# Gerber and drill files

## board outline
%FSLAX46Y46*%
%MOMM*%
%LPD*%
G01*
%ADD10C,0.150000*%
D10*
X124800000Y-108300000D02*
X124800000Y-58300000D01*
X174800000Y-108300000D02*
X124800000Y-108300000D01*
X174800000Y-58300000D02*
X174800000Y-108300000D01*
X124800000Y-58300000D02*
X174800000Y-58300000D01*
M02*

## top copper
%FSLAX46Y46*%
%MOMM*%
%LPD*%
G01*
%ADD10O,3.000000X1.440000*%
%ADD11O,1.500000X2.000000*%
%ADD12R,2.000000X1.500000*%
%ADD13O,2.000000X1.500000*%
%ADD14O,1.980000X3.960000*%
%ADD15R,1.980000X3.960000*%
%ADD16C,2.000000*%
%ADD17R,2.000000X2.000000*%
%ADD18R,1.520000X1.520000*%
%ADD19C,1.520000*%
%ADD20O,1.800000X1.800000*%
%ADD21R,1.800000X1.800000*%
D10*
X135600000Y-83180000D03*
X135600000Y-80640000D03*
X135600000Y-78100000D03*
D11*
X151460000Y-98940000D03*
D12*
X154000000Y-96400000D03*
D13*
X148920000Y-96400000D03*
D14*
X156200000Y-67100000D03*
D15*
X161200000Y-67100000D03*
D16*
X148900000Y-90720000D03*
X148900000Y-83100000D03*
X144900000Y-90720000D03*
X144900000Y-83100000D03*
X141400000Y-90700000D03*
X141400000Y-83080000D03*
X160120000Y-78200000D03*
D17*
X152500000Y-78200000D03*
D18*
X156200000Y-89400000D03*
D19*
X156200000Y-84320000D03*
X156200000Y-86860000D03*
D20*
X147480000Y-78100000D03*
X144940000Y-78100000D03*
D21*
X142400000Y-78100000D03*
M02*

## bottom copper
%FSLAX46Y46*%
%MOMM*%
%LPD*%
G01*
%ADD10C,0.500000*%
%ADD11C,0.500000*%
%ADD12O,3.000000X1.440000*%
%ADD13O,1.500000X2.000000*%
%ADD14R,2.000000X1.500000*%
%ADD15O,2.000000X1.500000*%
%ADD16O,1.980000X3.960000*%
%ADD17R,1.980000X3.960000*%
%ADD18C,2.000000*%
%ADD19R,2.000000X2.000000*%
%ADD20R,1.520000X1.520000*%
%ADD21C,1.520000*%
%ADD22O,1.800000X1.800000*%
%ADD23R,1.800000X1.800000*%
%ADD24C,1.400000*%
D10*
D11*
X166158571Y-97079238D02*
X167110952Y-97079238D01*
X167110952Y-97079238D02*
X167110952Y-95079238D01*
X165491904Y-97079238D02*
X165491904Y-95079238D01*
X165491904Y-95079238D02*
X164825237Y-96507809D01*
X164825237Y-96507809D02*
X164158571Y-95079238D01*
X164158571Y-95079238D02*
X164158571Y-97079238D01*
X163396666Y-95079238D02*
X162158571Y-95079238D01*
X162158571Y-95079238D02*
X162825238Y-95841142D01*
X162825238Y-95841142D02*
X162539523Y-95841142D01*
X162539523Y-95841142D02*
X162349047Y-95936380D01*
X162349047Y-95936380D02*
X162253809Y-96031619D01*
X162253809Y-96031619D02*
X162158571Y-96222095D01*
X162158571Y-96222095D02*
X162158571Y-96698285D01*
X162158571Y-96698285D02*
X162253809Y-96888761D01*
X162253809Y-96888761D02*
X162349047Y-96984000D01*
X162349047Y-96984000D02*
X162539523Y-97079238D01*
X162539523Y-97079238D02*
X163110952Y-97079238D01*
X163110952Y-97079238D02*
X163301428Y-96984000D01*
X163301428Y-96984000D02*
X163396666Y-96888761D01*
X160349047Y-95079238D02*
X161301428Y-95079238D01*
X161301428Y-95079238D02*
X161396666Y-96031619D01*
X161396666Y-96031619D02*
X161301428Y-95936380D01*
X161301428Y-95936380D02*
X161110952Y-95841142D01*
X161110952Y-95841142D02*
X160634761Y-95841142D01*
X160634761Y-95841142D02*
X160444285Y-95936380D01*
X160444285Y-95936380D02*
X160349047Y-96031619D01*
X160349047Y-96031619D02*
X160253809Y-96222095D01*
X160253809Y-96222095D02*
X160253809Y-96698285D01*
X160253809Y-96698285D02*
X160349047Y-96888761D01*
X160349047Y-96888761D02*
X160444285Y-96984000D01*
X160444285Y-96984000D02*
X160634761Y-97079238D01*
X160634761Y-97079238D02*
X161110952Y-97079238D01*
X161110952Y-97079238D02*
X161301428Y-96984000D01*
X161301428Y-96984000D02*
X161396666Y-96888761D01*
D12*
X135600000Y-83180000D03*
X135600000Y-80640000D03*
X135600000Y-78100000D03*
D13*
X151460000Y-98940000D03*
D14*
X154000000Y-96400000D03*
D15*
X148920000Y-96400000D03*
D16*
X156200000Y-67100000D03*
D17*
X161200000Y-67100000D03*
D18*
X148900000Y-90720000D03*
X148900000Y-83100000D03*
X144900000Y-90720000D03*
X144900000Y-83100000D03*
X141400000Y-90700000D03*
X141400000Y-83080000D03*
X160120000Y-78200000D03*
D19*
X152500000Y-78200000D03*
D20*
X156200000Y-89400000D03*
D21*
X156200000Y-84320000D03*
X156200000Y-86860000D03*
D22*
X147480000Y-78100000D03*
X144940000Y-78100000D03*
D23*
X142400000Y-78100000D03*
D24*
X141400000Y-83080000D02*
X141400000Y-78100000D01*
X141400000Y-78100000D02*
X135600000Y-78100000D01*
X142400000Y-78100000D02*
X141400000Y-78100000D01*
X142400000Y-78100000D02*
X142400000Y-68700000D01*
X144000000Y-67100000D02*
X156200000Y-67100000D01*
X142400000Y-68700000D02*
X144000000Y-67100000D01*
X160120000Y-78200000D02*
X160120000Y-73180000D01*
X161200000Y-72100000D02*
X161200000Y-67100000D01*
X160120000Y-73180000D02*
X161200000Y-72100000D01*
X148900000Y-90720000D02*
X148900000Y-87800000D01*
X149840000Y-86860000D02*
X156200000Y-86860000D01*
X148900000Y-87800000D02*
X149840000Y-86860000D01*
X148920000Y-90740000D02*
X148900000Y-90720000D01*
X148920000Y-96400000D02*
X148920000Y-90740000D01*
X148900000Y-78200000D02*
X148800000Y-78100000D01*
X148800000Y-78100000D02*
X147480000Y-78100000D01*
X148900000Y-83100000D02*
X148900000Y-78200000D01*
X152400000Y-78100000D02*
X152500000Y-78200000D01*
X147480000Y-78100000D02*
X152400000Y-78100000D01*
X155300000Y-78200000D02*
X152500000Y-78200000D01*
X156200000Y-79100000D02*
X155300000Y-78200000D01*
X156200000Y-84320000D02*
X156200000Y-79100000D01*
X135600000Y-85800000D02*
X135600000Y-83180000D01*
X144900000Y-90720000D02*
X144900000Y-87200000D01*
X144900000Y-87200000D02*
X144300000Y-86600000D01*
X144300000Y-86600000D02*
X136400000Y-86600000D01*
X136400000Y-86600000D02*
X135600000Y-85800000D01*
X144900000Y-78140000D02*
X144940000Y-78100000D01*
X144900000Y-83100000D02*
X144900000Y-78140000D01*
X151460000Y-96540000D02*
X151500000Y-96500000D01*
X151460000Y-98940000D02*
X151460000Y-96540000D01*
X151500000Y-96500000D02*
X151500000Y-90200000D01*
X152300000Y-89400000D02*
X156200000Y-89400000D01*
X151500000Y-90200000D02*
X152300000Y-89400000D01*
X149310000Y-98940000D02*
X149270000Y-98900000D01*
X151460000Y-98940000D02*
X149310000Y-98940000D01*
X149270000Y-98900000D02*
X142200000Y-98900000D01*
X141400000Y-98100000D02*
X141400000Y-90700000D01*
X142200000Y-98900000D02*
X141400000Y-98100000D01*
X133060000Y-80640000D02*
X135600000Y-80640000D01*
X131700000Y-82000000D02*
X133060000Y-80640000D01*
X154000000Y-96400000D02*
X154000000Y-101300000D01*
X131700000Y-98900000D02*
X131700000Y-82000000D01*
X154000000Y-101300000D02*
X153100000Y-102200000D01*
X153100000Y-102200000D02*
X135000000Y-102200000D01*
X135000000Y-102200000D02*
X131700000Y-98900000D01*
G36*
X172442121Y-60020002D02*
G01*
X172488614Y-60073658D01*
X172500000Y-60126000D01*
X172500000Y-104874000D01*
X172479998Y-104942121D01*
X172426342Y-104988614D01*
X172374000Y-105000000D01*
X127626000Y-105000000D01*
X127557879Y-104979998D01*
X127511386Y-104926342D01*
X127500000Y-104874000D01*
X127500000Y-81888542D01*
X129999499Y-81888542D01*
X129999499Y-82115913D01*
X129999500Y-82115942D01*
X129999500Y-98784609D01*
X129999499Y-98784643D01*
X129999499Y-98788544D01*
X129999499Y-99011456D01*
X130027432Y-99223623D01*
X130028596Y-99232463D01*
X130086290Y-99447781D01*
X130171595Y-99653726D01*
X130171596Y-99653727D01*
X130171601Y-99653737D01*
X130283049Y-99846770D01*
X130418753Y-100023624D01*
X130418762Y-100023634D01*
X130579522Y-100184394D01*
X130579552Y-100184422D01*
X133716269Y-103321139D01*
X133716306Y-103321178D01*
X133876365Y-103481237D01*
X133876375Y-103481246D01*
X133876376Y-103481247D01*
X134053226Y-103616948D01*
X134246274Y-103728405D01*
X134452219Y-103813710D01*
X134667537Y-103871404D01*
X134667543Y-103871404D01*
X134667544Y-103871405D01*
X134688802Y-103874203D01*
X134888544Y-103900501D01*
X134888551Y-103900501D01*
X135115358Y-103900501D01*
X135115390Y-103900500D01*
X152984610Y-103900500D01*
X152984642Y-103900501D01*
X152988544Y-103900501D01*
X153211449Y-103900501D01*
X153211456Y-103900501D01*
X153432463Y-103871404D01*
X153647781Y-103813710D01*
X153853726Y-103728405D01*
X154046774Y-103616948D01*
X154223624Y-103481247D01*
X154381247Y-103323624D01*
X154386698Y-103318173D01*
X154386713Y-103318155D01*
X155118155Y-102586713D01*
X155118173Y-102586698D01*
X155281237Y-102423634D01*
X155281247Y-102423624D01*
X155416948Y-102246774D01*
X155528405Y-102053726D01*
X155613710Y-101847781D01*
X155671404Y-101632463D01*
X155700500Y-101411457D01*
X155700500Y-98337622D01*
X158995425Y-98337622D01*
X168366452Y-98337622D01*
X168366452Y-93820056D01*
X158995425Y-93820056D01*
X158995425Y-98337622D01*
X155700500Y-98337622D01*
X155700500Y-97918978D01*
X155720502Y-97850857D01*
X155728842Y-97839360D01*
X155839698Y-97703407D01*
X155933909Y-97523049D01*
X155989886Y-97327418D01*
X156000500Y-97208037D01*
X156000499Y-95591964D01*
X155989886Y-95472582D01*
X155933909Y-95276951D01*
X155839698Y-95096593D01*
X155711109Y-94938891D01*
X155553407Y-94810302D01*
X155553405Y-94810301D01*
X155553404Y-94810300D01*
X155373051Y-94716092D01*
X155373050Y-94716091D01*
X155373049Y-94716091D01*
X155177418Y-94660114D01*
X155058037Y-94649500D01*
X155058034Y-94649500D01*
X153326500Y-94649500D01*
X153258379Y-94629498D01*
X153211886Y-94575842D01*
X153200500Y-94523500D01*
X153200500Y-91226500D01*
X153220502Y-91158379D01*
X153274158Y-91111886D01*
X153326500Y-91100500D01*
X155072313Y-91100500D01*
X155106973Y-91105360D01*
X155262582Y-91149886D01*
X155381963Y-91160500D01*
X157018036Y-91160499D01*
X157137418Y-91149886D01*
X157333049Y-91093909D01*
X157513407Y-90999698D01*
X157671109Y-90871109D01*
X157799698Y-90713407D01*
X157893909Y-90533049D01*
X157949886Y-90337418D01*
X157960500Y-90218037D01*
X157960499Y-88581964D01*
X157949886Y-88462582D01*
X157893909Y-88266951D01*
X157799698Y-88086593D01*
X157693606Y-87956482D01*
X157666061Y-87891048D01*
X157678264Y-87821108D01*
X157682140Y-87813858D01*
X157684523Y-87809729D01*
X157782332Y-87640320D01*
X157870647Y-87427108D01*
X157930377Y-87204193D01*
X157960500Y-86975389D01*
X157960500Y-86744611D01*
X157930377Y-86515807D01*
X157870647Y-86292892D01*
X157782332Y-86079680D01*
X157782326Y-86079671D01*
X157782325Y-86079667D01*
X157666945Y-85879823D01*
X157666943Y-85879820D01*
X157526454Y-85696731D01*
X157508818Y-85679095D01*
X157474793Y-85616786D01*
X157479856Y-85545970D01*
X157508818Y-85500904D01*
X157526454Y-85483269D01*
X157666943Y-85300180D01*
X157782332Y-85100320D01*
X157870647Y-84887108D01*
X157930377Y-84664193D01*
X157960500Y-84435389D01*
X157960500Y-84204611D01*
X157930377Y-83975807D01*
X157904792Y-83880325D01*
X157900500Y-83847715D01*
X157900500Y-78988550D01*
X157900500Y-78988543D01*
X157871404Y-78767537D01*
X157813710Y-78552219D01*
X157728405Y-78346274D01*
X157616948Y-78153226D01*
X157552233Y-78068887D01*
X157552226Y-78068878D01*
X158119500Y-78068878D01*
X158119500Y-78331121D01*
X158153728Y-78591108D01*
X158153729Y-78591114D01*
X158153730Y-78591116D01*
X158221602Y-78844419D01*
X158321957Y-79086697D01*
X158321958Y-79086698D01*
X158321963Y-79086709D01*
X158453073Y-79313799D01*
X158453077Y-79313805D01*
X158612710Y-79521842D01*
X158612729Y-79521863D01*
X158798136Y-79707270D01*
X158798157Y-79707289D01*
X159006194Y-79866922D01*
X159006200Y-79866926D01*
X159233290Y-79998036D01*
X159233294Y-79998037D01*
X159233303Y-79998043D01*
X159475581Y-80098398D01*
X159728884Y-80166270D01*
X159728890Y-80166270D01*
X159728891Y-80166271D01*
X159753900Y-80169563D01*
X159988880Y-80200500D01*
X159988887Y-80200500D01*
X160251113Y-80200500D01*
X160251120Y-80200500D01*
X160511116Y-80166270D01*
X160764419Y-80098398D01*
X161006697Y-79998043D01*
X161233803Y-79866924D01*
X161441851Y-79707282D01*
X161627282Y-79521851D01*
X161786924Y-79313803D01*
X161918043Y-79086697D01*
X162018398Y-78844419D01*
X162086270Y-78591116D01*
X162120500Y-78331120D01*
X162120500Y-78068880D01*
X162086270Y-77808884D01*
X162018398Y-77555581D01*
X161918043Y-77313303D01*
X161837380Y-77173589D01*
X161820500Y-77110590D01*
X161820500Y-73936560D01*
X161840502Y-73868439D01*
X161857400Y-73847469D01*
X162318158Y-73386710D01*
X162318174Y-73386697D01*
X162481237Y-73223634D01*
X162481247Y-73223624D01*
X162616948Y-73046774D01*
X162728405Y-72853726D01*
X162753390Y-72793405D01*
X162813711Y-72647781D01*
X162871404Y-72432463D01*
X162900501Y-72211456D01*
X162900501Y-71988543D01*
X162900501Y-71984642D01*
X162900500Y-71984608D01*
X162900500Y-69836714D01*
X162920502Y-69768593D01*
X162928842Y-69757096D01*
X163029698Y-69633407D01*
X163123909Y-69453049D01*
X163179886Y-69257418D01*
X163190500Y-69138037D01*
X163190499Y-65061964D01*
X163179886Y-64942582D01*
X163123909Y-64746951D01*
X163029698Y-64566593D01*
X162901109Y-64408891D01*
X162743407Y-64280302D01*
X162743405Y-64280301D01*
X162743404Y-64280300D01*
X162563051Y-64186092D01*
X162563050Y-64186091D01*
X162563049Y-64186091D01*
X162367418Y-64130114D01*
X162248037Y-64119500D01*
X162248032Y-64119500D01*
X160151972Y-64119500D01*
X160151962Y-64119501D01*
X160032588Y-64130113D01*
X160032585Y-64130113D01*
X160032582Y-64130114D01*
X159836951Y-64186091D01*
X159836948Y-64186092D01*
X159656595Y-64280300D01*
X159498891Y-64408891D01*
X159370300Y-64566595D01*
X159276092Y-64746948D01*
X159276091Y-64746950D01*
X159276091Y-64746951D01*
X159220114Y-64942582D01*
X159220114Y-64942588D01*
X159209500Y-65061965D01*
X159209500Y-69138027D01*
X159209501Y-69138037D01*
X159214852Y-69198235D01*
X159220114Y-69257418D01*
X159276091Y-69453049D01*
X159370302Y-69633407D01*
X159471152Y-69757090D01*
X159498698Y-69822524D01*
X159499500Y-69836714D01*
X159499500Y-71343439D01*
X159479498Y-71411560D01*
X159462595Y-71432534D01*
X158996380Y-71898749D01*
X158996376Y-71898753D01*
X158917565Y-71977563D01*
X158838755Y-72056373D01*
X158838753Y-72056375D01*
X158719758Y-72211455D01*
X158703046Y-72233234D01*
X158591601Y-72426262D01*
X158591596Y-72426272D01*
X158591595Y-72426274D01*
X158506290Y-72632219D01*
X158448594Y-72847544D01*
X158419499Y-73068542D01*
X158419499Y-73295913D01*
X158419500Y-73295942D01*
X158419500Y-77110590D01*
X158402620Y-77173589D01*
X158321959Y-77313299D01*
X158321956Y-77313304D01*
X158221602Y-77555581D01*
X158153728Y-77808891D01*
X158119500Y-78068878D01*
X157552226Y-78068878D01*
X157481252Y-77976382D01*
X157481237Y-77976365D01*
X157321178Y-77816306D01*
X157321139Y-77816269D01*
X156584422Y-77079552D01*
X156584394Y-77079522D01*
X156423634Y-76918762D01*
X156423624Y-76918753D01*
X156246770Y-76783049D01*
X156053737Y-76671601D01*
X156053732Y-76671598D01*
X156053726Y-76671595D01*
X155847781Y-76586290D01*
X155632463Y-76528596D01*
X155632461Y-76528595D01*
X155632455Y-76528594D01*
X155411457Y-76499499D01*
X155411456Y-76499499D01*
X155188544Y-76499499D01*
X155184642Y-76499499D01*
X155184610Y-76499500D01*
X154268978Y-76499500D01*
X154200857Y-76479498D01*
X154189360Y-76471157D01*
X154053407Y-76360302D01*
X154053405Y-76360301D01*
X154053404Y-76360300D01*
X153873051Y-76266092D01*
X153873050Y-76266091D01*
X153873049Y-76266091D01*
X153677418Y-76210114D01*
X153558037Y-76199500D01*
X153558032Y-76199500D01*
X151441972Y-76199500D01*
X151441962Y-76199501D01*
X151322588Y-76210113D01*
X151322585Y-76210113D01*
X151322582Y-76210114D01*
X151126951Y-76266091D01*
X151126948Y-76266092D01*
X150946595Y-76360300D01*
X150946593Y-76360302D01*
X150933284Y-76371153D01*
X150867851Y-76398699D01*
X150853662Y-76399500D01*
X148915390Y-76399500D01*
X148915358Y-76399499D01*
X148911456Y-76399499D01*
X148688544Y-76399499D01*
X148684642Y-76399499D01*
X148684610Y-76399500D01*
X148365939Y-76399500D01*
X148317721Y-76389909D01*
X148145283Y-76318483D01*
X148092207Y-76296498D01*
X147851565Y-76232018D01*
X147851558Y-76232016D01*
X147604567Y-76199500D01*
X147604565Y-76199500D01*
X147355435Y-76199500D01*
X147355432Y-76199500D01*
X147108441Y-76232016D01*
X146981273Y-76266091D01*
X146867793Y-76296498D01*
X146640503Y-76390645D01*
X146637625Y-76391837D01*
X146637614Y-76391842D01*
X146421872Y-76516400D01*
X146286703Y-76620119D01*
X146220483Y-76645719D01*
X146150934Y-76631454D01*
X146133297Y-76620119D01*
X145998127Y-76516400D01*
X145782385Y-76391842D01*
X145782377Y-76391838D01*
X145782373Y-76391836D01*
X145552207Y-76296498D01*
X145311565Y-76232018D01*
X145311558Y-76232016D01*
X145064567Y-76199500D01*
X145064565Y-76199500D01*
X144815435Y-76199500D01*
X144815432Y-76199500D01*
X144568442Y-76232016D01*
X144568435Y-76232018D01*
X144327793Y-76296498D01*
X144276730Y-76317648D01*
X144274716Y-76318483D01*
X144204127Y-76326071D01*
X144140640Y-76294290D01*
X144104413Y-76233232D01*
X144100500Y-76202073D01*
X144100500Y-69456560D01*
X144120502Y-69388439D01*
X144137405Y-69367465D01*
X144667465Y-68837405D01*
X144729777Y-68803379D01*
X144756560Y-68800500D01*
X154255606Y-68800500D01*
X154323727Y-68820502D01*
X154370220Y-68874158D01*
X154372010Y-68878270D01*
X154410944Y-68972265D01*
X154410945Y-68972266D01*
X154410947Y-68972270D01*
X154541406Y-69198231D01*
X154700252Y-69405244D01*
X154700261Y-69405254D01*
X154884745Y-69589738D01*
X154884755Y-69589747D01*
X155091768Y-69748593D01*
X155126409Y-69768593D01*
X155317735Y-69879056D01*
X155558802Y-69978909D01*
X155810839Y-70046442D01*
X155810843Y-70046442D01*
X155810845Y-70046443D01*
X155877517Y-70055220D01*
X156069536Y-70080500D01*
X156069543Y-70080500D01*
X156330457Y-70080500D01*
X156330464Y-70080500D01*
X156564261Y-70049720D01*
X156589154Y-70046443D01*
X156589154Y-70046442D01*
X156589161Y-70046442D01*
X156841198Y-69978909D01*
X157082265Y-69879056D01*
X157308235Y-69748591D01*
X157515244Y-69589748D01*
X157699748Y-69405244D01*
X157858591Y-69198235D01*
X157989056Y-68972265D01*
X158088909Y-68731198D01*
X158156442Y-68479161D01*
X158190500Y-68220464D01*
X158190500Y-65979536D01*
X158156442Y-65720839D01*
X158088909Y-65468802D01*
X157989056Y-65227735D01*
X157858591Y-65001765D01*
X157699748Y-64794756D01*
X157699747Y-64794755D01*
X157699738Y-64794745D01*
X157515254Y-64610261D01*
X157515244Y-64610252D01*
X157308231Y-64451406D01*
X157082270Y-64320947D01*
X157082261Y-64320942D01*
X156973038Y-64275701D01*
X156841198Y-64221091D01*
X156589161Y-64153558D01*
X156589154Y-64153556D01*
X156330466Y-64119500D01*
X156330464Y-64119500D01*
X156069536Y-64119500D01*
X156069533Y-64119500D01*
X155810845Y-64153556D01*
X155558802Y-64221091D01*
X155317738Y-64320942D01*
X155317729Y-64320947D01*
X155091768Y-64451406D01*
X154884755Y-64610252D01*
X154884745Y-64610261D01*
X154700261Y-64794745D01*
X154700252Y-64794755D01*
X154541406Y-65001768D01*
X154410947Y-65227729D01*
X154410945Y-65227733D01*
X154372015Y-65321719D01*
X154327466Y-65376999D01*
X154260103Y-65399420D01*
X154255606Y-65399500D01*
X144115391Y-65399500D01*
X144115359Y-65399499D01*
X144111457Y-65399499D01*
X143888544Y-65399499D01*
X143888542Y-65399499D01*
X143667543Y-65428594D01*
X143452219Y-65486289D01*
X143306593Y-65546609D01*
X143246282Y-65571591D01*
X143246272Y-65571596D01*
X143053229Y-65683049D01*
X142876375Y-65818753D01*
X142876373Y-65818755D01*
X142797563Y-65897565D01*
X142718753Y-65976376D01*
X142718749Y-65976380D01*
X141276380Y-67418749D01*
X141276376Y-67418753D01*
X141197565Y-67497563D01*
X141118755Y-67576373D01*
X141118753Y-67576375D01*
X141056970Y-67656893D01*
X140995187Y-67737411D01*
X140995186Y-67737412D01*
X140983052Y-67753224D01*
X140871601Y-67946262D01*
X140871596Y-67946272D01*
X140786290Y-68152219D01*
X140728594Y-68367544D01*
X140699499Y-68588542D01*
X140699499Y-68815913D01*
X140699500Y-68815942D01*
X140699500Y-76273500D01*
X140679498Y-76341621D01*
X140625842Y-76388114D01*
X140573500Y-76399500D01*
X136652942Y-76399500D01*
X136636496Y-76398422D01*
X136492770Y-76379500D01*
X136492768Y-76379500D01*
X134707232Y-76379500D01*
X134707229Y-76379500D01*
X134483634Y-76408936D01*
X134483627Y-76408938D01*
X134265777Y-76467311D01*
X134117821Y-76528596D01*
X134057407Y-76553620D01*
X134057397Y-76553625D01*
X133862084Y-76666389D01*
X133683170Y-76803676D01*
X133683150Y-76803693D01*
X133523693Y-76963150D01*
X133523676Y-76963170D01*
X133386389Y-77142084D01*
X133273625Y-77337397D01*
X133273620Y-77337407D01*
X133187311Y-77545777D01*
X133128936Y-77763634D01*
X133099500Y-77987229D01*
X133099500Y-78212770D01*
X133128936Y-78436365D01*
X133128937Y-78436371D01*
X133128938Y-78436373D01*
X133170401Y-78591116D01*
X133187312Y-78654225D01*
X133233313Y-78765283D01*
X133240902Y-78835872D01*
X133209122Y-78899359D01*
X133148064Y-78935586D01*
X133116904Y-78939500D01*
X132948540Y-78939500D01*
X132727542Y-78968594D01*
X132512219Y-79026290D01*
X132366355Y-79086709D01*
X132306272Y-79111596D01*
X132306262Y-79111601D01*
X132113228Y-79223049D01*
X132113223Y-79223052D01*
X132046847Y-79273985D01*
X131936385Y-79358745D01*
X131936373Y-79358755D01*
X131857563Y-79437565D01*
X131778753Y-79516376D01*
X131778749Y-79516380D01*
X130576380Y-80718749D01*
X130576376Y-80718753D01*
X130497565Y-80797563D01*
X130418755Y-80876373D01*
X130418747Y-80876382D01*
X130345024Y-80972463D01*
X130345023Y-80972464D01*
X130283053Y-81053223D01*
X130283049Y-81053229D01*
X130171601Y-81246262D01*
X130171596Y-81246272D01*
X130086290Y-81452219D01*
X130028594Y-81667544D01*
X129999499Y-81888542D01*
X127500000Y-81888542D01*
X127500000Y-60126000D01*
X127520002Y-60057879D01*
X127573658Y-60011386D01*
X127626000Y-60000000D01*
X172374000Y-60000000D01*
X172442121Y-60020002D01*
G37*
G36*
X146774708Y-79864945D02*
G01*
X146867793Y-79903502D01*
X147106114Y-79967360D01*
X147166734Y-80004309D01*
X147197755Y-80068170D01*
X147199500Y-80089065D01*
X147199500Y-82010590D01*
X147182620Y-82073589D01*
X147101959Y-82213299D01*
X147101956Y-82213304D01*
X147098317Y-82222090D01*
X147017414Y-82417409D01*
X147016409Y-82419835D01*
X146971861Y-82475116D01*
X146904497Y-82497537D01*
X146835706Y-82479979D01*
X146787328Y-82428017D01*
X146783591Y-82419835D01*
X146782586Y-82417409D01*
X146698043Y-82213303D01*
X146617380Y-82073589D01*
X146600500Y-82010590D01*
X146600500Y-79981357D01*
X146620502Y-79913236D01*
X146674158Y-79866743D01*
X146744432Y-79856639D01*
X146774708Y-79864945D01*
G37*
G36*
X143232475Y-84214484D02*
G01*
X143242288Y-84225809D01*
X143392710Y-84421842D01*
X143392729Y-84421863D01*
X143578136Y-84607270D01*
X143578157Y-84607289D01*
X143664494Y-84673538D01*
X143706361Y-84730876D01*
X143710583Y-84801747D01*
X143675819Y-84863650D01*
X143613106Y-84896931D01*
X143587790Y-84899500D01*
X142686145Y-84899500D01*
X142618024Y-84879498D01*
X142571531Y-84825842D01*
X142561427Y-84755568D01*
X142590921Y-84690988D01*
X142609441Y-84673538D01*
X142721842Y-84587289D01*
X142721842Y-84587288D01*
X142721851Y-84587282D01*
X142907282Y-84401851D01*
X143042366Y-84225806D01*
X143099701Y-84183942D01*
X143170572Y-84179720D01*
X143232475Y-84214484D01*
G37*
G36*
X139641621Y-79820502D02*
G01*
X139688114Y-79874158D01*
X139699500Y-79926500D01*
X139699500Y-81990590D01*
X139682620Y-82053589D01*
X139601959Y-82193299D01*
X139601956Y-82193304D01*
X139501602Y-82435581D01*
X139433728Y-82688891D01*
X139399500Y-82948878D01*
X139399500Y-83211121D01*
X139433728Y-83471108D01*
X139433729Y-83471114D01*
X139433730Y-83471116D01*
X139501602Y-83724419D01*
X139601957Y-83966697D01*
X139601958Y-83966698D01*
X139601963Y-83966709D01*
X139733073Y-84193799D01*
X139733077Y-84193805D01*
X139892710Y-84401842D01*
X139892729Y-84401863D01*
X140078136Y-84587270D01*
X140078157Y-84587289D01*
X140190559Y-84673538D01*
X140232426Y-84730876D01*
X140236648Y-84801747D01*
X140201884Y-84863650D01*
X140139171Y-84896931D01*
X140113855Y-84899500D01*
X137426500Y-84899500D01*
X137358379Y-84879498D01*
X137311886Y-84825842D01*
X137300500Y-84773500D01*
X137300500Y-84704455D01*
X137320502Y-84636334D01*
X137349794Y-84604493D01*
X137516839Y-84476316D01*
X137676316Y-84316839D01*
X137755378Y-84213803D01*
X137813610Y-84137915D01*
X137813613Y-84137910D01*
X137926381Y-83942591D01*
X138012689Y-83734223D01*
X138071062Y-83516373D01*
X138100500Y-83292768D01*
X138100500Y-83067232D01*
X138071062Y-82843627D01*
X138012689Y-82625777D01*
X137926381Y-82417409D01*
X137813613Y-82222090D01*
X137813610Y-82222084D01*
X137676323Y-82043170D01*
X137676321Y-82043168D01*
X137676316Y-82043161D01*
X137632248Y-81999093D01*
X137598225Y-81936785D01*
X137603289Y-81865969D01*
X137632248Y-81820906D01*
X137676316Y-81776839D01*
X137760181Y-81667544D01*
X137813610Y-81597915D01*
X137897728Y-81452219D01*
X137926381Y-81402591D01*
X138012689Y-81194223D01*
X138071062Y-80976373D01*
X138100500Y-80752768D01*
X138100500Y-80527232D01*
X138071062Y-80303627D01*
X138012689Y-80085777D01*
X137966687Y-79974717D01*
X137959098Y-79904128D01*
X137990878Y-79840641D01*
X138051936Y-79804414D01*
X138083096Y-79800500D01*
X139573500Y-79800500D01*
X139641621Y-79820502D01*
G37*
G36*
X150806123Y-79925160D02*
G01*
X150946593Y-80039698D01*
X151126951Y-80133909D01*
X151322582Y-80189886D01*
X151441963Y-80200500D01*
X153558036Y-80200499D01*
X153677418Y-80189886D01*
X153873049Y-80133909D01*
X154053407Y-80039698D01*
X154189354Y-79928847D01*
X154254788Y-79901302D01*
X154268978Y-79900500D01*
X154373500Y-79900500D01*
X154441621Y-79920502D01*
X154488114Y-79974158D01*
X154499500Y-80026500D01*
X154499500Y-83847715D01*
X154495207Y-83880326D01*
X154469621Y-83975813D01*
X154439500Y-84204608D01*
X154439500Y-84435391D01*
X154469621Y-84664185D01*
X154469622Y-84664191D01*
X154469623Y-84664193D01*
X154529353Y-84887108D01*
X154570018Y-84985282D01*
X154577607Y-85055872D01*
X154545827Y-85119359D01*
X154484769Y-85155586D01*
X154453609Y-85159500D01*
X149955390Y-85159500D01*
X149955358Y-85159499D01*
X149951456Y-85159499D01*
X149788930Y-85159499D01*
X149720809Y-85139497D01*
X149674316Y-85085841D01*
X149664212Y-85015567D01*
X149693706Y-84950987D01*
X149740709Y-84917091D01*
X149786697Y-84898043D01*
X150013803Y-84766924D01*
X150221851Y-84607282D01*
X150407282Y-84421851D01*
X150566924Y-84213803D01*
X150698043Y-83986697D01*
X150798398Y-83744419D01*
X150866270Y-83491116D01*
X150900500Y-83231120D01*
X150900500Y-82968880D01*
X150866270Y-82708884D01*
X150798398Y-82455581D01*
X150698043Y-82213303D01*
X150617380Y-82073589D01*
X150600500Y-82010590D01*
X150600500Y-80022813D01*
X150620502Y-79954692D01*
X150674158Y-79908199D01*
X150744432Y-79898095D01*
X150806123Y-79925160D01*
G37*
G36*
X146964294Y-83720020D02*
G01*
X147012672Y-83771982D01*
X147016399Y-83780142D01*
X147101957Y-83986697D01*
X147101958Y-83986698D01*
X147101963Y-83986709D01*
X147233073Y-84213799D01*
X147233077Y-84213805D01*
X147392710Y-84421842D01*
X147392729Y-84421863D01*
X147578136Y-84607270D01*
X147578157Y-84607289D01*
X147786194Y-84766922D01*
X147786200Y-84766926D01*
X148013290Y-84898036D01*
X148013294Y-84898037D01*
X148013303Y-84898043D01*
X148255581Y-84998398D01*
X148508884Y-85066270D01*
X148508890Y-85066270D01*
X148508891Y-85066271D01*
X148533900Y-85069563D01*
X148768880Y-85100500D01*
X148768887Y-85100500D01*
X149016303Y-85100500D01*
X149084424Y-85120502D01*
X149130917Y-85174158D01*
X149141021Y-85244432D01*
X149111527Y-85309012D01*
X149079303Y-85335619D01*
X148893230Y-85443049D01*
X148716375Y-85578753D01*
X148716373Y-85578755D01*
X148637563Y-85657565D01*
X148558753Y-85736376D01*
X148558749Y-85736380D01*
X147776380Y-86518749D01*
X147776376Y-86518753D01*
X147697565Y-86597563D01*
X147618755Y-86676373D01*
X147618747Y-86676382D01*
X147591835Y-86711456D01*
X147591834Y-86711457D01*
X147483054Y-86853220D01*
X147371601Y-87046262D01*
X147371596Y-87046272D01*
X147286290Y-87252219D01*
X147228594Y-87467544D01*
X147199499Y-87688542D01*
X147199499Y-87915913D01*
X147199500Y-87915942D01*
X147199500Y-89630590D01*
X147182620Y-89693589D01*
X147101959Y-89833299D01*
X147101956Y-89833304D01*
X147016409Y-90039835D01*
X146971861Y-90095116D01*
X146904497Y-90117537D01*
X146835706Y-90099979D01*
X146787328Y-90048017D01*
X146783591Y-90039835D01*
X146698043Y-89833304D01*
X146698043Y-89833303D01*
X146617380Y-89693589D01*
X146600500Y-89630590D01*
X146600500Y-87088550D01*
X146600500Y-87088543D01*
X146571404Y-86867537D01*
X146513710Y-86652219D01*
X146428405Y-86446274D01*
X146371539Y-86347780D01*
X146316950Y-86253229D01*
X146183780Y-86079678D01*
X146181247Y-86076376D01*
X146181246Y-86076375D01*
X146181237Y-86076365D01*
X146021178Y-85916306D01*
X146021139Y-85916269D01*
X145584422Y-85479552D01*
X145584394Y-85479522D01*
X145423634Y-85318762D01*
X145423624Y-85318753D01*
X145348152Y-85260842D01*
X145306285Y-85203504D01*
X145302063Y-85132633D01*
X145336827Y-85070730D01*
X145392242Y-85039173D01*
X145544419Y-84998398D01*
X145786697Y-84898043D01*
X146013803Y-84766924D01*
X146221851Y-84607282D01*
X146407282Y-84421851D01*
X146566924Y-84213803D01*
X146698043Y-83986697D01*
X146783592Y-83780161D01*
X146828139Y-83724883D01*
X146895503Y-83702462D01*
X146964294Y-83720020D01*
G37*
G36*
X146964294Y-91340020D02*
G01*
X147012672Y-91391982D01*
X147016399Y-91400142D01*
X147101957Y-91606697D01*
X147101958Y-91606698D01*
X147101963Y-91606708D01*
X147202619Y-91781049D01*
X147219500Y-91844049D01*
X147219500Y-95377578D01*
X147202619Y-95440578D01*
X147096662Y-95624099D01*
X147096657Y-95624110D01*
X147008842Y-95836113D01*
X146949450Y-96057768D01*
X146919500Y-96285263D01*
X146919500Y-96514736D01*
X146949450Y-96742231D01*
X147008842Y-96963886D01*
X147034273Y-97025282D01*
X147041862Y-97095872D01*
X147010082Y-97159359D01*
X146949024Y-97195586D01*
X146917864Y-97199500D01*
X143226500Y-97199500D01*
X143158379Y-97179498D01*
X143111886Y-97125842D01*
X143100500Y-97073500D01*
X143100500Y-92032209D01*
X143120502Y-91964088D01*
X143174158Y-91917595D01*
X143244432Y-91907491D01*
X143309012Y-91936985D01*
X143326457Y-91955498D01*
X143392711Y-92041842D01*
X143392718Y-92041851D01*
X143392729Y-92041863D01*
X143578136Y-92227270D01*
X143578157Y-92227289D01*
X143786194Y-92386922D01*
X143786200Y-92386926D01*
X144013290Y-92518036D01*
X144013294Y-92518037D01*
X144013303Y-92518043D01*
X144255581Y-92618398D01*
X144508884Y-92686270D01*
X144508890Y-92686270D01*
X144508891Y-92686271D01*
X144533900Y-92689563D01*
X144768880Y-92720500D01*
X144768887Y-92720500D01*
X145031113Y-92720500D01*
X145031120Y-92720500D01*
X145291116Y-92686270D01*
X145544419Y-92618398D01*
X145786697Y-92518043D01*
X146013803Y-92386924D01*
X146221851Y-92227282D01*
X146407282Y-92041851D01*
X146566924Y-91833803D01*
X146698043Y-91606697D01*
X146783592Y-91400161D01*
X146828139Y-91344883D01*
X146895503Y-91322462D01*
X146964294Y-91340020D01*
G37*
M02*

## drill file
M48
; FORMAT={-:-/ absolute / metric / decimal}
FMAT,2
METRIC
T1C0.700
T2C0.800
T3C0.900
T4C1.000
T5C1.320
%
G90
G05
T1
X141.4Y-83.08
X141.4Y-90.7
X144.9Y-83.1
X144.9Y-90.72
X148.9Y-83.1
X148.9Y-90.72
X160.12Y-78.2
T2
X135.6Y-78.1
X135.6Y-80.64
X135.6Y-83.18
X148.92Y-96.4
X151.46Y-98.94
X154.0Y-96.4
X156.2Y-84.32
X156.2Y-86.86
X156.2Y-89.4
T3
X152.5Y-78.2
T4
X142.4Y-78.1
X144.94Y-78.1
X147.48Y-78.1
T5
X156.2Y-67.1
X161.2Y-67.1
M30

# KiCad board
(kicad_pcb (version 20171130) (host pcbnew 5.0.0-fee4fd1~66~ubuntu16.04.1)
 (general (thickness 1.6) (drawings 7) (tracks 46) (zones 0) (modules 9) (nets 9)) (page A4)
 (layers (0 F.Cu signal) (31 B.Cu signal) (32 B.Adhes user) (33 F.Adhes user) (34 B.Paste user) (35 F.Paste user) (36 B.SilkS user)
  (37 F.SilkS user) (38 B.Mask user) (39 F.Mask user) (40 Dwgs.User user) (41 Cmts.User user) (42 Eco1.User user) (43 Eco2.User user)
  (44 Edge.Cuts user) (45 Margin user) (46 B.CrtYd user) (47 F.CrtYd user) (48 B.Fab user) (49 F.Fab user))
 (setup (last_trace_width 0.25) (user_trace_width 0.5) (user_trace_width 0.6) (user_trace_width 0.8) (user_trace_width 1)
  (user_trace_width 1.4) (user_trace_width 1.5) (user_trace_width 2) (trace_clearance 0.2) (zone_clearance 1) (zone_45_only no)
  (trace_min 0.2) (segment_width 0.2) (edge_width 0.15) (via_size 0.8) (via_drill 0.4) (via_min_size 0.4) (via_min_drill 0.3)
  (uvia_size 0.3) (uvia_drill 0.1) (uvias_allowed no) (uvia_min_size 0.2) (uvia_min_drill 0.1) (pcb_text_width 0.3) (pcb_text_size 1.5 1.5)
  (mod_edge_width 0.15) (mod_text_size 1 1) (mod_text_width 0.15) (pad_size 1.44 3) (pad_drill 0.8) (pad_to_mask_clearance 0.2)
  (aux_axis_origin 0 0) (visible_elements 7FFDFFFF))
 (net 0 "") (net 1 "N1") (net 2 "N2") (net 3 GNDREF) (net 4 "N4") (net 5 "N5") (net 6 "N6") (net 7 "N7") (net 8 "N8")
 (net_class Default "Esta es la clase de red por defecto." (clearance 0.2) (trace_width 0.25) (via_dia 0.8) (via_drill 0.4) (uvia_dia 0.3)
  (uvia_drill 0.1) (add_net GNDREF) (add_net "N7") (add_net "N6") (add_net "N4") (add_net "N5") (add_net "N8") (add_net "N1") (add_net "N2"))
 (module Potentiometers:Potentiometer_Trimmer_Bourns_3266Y (layer F.Cu) (at 135.6 78.1 90)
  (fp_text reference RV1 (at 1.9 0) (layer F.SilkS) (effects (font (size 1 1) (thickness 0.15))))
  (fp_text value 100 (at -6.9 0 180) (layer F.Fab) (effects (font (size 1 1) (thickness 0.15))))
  (pad 3 thru_hole oval (at -5.08 0 90) (size 1.44 3) (drill 0.8) (layers *.Cu *.Mask) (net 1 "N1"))
  (pad 2 thru_hole oval (at -2.54 0 90) (size 1.44 3) (drill 0.8) (layers *.Cu *.Mask) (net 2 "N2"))
  (pad 1 thru_hole oval (at 0 0 90) (size 1.44 3) (drill 0.8) (layers *.Cu *.Mask) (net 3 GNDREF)))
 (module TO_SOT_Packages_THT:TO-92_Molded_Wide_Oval (layer F.Cu) (at 154 96.4 180)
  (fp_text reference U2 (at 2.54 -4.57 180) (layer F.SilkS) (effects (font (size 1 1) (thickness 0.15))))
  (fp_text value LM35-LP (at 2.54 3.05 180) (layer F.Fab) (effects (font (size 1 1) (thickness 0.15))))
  (pad 2 thru_hole oval (at 2.54 -2.54 270) (size 2 1.5) (drill 0.8) (layers *.Cu *.Mask) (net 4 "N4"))
  (pad 1 thru_hole rect (at 0 0 270) (size 1.5 2) (drill 0.8) (layers *.Cu *.Mask) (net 2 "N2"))
  (pad 3 thru_hole oval (at 5.08 0 270) (size 1.5 2) (drill 0.8) (layers *.Cu *.Mask) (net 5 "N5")))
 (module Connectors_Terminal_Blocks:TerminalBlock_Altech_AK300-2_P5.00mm (layer F.Cu) (at 161.2 67.1 180)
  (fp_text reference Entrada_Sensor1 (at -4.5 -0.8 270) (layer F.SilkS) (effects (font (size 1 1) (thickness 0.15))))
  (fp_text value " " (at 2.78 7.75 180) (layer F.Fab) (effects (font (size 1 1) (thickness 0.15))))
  (pad 2 thru_hole oval (at 5 0 180) (size 1.98 3.96) (drill 1.32) (layers *.Cu *.Mask) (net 3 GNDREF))
  (pad 1 thru_hole rect (at 0 0 180) (size 1.98 3.96) (drill 1.32) (layers *.Cu *.Mask) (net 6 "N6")))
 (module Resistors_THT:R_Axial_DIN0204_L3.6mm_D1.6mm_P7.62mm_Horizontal (layer F.Cu) (at 148.9 83.1 270)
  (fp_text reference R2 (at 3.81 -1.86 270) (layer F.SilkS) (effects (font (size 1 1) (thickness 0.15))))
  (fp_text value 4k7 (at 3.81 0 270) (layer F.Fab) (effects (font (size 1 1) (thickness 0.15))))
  (pad 2 thru_hole circle (at 7.62 0 270) (size 2 2) (drill 0.7) (layers *.Cu *.Mask) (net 5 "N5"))
  (pad 1 thru_hole circle (at 0 0 270) (size 2 2) (drill 0.7) (layers *.Cu *.Mask) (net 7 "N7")))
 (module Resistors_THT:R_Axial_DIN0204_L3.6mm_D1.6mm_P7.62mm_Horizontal (layer F.Cu) (at 144.9 83.1 270)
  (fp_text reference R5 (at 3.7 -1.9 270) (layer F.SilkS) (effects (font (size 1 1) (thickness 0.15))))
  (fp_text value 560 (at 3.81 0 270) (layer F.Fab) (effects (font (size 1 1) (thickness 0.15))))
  (pad 2 thru_hole circle (at 7.62 0 270) (size 2 2) (drill 0.7) (layers *.Cu *.Mask) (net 1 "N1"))
  (pad 1 thru_hole circle (at 0 0 270) (size 2 2) (drill 0.7) (layers *.Cu *.Mask) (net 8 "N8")))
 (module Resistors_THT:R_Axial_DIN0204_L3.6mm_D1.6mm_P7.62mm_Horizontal (layer F.Cu) (at 141.4 90.7 90)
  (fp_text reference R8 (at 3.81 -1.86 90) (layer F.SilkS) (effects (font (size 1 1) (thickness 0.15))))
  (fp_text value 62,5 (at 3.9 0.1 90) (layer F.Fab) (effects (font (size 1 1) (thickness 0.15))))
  (pad 1 thru_hole circle (at 0 0 90) (size 2 2) (drill 0.7) (layers *.Cu *.Mask) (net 4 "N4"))
  (pad 2 thru_hole circle (at 7.62 0 90) (size 2 2) (drill 0.7) (layers *.Cu *.Mask) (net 3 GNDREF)))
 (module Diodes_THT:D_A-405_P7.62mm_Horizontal (layer F.Cu) (at 152.5 78.2)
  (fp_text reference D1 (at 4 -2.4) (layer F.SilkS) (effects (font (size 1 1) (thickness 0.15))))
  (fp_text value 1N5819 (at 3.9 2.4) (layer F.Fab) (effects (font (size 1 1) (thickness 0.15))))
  (pad 2 thru_hole circle (at 7.62 0) (size 2 2) (drill 0.7) (layers *.Cu *.Mask) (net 6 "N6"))
  (pad 1 thru_hole rect (at 0 0) (size 2 2) (drill 0.9) (layers *.Cu *.Mask) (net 7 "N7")))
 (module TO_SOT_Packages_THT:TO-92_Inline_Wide (layer F.Cu) (at 156.2 89.4 90)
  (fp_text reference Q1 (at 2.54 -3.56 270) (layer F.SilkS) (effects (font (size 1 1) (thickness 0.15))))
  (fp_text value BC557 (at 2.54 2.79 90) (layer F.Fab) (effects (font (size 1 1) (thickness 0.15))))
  (pad 1 thru_hole rect (at 0 0 180) (size 1.52 1.52) (drill 0.8) (layers *.Cu *.Mask) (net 4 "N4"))
  (pad 3 thru_hole circle (at 5.08 0 180) (size 1.52 1.52) (drill 0.8) (layers *.Cu *.Mask) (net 7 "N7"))
  (pad 2 thru_hole circle (at 2.54 0 180) (size 1.52 1.52) (drill 0.8) (layers *.Cu *.Mask) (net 5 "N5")))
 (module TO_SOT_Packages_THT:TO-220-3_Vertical (layer F.Cu) (at 142.4 78.1)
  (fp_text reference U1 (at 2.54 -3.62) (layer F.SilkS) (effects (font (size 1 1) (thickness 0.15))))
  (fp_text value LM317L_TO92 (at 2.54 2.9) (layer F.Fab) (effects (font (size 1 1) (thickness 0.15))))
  (pad 3 thru_hole oval (at 5.08 0) (size 1.8 1.8) (drill 1) (layers *.Cu *.Mask) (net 7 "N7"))
  (pad 2 thru_hole oval (at 2.54 0) (size 1.8 1.8) (drill 1) (layers *.Cu *.Mask) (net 8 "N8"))
  (pad 1 thru_hole rect (at 0 0) (size 1.8 1.8) (drill 1) (layers *.Cu *.Mask) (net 3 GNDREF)))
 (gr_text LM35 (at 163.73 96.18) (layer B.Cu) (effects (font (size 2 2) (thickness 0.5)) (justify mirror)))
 (gr_line (start 124.8 108.3) (end 124.8 58.3) (layer Edge.Cuts) (width 0.15))
 (gr_line (start 174.8 108.3) (end 124.8 108.3) (layer Edge.Cuts) (width 0.15))
 (gr_line (start 174.8 58.3) (end 174.8 108.3) (layer Edge.Cuts) (width 0.15))
 (gr_line (start 124.8 58.3) (end 174.8 58.3) (layer Edge.Cuts) (width 0.15))
 (segment (start 141.4 83.08) (end 141.4 78.1) (width 1.4) (layer B.Cu) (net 3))
 (segment (start 141.4 78.1) (end 135.6 78.1) (width 1.4) (layer B.Cu) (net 3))
 (segment (start 142.4 78.1) (end 141.4 78.1) (width 1.4) (layer B.Cu) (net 3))
 (segment (start 142.4 78.1) (end 142.4 68.7) (width 1.4) (layer B.Cu) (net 3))
 (segment (start 144 67.1) (end 156.2 67.1) (width 1.4) (layer B.Cu) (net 3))
 (segment (start 142.4 68.7) (end 144 67.1) (width 1.4) (layer B.Cu) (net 3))
 (segment (start 160.12 78.2) (end 160.12 73.18) (width 1.4) (layer B.Cu) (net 6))
 (segment (start 161.2 72.1) (end 161.2 67.1) (width 1.4) (layer B.Cu) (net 6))
 (segment (start 160.12 73.18) (end 161.2 72.1) (width 1.4) (layer B.Cu) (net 6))
 (segment (start 148.9 90.72) (end 148.9 87.8) (width 1.4) (layer B.Cu) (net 5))
 (segment (start 149.84 86.86) (end 156.2 86.86) (width 1.4) (layer B.Cu) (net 5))
 (segment (start 148.9 87.8) (end 149.84 86.86) (width 1.4) (layer B.Cu) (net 5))
 (segment (start 148.92 90.74) (end 148.9 90.72) (width 1.4) (layer B.Cu) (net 5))
 (segment (start 148.92 96.4) (end 148.92 90.74) (width 1.4) (layer B.Cu) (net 5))
 (segment (start 148.9 78.2) (end 148.8 78.1) (width 1.4) (layer B.Cu) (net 7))
 (segment (start 148.8 78.1) (end 147.48 78.1) (width 1.4) (layer B.Cu) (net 7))
 (segment (start 148.9 83.1) (end 148.9 78.2) (width 1.4) (layer B.Cu) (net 7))
 (segment (start 152.4 78.1) (end 152.5 78.2) (width 1.4) (layer B.Cu) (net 7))
 (segment (start 147.48 78.1) (end 152.4 78.1) (width 1.4) (layer B.Cu) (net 7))
 (segment (start 155.3 78.2) (end 152.5 78.2) (width 1.4) (layer B.Cu) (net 7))
 (segment (start 156.2 79.1) (end 155.3 78.2) (width 1.4) (layer B.Cu) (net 7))
 (segment (start 156.2 84.32) (end 156.2 79.1) (width 1.4) (layer B.Cu) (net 7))
 (segment (start 135.6 85.8) (end 135.6 83.18) (width 1.4) (layer B.Cu) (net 1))
 (segment (start 144.9 90.72) (end 144.9 87.2) (width 1.4) (layer B.Cu) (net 1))
 (segment (start 144.9 87.2) (end 144.3 86.6) (width 1.4) (layer B.Cu) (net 1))
 (segment (start 144.3 86.6) (end 136.4 86.6) (width 1.4) (layer B.Cu) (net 1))
 (segment (start 136.4 86.6) (end 135.6 85.8) (width 1.4) (layer B.Cu) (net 1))
 (segment (start 144.9 78.14) (end 144.94 78.1) (width 1.4) (layer B.Cu) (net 8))
 (segment (start 144.9 83.1) (end 144.9 78.14) (width 1.4) (layer B.Cu) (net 8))
 (segment (start 151.46 96.54) (end 151.5 96.5) (width 1.4) (layer B.Cu) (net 4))
 (segment (start 151.46 98.94) (end 151.46 96.54) (width 1.4) (layer B.Cu) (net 4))
 (segment (start 151.5 96.5) (end 151.5 90.2) (width 1.4) (layer B.Cu) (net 4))
 (segment (start 152.3 89.4) (end 156.2 89.4) (width 1.4) (layer B.Cu) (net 4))
 (segment (start 151.5 90.2) (end 152.3 89.4) (width 1.4) (layer B.Cu) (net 4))
 (segment (start 149.31 98.94) (end 149.27 98.9) (width 1.4) (layer B.Cu) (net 4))
 (segment (start 151.46 98.94) (end 149.31 98.94) (width 1.4) (layer B.Cu) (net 4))
 (segment (start 149.27 98.9) (end 142.2 98.9) (width 1.4) (layer B.Cu) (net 4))
 (segment (start 141.4 98.1) (end 141.4 90.7) (width 1.4) (layer B.Cu) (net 4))
 (segment (start 142.2 98.9) (end 141.4 98.1) (width 1.4) (layer B.Cu) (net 4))
 (segment (start 133.06 80.64) (end 135.6 80.64) (width 1.4) (layer B.Cu) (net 2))
 (segment (start 131.7 82) (end 133.06 80.64) (width 1.4) (layer B.Cu) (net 2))
 (segment (start 154 96.4) (end 154 101.3) (width 1.4) (layer B.Cu) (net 2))
 (segment (start 131.7 98.9) (end 131.7 82) (width 1.4) (layer B.Cu) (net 2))
 (segment (start 154 101.3) (end 153.1 102.2) (width 1.4) (layer B.Cu) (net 2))
 (segment (start 153.1 102.2) (end 135 102.2) (width 1.4) (layer B.Cu) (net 2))
 (segment (start 135 102.2) (end 131.7 98.9) (width 1.4) (layer B.Cu) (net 2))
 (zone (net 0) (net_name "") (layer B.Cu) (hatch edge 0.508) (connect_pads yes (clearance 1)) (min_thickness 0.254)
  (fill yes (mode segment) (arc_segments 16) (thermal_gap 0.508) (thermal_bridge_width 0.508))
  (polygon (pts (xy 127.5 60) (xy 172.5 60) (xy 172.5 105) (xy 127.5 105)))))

